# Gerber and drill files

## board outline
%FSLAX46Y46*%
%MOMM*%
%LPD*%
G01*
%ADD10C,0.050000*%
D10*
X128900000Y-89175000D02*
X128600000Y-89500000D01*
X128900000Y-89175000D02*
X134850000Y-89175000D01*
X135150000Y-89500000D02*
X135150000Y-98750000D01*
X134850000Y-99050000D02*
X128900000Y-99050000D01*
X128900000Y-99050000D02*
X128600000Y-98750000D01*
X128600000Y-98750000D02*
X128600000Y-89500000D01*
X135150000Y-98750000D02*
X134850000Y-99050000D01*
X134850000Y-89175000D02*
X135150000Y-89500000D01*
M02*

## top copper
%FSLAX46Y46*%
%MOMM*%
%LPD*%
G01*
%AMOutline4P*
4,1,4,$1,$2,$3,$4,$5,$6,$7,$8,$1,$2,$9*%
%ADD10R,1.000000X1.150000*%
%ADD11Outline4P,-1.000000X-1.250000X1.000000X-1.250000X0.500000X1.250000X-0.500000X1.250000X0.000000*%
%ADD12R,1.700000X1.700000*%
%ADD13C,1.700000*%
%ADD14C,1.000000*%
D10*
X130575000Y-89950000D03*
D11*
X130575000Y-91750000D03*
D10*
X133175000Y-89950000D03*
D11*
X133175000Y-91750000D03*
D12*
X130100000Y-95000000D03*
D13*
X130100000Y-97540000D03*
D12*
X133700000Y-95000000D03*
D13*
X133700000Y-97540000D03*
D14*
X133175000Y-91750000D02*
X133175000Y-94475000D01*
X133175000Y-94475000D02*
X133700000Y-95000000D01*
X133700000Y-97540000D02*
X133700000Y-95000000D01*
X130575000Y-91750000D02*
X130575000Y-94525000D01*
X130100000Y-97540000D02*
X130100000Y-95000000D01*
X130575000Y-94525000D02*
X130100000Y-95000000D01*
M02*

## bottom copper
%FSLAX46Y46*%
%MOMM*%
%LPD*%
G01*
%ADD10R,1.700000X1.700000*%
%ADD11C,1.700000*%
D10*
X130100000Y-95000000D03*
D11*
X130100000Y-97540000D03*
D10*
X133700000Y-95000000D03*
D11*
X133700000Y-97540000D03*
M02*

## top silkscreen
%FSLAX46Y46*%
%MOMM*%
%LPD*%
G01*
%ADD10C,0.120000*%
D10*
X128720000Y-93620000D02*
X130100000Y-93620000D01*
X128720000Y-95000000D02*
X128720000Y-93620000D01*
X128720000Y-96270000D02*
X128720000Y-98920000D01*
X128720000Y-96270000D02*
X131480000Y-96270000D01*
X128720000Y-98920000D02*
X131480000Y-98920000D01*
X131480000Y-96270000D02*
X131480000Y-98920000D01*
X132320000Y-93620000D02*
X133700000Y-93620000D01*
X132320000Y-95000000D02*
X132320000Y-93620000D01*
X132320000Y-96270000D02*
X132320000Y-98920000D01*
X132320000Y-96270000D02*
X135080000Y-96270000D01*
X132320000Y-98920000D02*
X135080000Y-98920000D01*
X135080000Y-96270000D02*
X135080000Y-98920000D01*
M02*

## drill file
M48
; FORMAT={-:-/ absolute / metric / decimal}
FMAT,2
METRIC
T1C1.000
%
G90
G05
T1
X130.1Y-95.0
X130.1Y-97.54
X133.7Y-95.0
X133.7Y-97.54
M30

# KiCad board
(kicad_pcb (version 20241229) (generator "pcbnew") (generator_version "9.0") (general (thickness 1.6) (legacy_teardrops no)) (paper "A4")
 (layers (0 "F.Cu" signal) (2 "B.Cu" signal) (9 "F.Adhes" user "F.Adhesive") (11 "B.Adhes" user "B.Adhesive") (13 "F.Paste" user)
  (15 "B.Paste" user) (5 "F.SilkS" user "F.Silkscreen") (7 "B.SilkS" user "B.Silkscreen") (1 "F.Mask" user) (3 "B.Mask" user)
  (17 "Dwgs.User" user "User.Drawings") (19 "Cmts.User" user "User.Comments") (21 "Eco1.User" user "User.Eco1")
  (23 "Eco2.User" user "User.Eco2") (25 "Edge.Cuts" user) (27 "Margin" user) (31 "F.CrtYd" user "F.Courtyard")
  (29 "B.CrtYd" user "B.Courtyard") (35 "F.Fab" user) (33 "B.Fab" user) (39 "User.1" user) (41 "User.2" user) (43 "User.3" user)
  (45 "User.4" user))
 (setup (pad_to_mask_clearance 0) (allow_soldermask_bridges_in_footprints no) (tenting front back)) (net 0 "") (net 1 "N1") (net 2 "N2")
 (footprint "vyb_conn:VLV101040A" (layer "F.Cu") (at 131.875 89.95)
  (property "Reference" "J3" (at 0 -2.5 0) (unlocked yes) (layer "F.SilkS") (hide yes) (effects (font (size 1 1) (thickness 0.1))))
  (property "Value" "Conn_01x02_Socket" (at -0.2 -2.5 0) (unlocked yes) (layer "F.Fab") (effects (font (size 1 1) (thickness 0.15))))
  (pad "1" smd rect (at -1.3 0) (size 1 1.15) (layers "F.Cu" "F.Mask" "F.Paste") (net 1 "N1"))
  (pad "1" smd trapezoid (at -1.3 1.8) (size 1.5 2.5) (rect_delta 0 0.5) (layers "F.Cu" "F.Mask" "F.Paste") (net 1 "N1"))
  (pad "2" smd rect (at 1.3 0) (size 1 1.15) (layers "F.Cu" "F.Mask" "F.Paste") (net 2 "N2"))
  (pad "2" smd trapezoid (at 1.3 1.8) (size 1.5 2.5) (rect_delta 0 0.5) (layers "F.Cu" "F.Mask" "F.Paste") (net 2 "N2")))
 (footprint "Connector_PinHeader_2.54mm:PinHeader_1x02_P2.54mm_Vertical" (layer "F.Cu") (at 130.1 95)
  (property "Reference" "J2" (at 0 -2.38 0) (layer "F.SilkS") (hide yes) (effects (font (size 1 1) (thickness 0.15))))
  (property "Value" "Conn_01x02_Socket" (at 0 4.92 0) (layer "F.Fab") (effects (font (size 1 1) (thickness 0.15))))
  (fp_line (start -1.38 -1.38) (end 0 -1.38) (stroke (width 0.12) (type solid)) (layer "F.SilkS"))
  (fp_line (start -1.38 0) (end -1.38 -1.38) (stroke (width 0.12) (type solid)) (layer "F.SilkS"))
  (fp_line (start -1.38 1.27) (end -1.38 3.92) (stroke (width 0.12) (type solid)) (layer "F.SilkS"))
  (fp_line (start -1.38 1.27) (end 1.38 1.27) (stroke (width 0.12) (type solid)) (layer "F.SilkS"))
  (fp_line (start -1.38 3.92) (end 1.38 3.92) (stroke (width 0.12) (type solid)) (layer "F.SilkS"))
  (fp_line (start 1.38 1.27) (end 1.38 3.92) (stroke (width 0.12) (type solid)) (layer "F.SilkS"))
  (pad "1" thru_hole rect (at 0 0) (size 1.7 1.7) (drill 1) (layers "*.Cu" "*.Mask") (remove_unused_layers no) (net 1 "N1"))
  (pad "2" thru_hole circle (at 0 2.54) (size 1.7 1.7) (drill 1) (layers "*.Cu" "*.Mask") (remove_unused_layers no) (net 1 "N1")))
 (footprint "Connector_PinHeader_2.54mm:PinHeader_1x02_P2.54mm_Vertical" (layer "F.Cu") (at 133.7 95)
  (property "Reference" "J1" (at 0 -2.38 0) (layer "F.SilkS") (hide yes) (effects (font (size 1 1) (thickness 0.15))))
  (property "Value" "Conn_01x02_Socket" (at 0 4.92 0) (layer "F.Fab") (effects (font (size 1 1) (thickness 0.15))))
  (fp_line (start -1.38 -1.38) (end 0 -1.38) (stroke (width 0.12) (type solid)) (layer "F.SilkS"))
  (fp_line (start -1.38 0) (end -1.38 -1.38) (stroke (width 0.12) (type solid)) (layer "F.SilkS"))
  (fp_line (start -1.38 1.27) (end -1.38 3.92) (stroke (width 0.12) (type solid)) (layer "F.SilkS"))
  (fp_line (start -1.38 1.27) (end 1.38 1.27) (stroke (width 0.12) (type solid)) (layer "F.SilkS"))
  (fp_line (start -1.38 3.92) (end 1.38 3.92) (stroke (width 0.12) (type solid)) (layer "F.SilkS"))
  (fp_line (start 1.38 1.27) (end 1.38 3.92) (stroke (width 0.12) (type solid)) (layer "F.SilkS"))
  (pad "1" thru_hole rect (at 0 0) (size 1.7 1.7) (drill 1) (layers "*.Cu" "*.Mask") (remove_unused_layers no) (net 2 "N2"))
  (pad "2" thru_hole circle (at 0 2.54) (size 1.7 1.7) (drill 1) (layers "*.Cu" "*.Mask") (remove_unused_layers no) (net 2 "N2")))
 (gr_line (start 128.9 89.175) (end 128.6 89.5) (stroke (width 0.05) (type default)) (layer "Edge.Cuts"))
 (gr_line (start 128.9 89.175) (end 134.85 89.175) (stroke (width 0.05) (type default)) (layer "Edge.Cuts"))
 (gr_line (start 135.15 89.5) (end 135.15 98.75) (stroke (width 0.05) (type default)) (layer "Edge.Cuts"))
 (gr_line (start 134.85 99.05) (end 128.9 99.05) (stroke (width 0.05) (type default)) (layer "Edge.Cuts"))
 (gr_line (start 128.9 99.05) (end 128.6 98.75) (stroke (width 0.05) (type default)) (layer "Edge.Cuts"))
 (gr_line (start 128.6 98.75) (end 128.6 89.5) (stroke (width 0.05) (type default)) (layer "Edge.Cuts"))
 (gr_line (start 135.15 98.75) (end 134.85 99.05) (stroke (width 0.05) (type default)) (layer "Edge.Cuts"))
 (gr_line (start 134.85 89.175) (end 135.15 89.5) (stroke (width 0.05) (type default)) (layer "Edge.Cuts"))
 (segment (start 133.175 91.75) (end 133.175 94.475) (width 1) (layer "F.Cu") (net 2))
 (segment (start 133.175 94.475) (end 133.7 95) (width 1) (layer "F.Cu") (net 2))
 (segment (start 133.7 97.54) (end 133.7 95) (width 1) (layer "F.Cu") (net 2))
 (segment (start 130.575 91.75) (end 130.575 94.525) (width 1) (layer "F.Cu") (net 1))
 (segment (start 130.1 97.54) (end 130.1 95) (width 1) (layer "F.Cu") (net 1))
 (segment (start 130.575 94.525) (end 130.1 95) (width 1) (layer "F.Cu") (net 1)))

